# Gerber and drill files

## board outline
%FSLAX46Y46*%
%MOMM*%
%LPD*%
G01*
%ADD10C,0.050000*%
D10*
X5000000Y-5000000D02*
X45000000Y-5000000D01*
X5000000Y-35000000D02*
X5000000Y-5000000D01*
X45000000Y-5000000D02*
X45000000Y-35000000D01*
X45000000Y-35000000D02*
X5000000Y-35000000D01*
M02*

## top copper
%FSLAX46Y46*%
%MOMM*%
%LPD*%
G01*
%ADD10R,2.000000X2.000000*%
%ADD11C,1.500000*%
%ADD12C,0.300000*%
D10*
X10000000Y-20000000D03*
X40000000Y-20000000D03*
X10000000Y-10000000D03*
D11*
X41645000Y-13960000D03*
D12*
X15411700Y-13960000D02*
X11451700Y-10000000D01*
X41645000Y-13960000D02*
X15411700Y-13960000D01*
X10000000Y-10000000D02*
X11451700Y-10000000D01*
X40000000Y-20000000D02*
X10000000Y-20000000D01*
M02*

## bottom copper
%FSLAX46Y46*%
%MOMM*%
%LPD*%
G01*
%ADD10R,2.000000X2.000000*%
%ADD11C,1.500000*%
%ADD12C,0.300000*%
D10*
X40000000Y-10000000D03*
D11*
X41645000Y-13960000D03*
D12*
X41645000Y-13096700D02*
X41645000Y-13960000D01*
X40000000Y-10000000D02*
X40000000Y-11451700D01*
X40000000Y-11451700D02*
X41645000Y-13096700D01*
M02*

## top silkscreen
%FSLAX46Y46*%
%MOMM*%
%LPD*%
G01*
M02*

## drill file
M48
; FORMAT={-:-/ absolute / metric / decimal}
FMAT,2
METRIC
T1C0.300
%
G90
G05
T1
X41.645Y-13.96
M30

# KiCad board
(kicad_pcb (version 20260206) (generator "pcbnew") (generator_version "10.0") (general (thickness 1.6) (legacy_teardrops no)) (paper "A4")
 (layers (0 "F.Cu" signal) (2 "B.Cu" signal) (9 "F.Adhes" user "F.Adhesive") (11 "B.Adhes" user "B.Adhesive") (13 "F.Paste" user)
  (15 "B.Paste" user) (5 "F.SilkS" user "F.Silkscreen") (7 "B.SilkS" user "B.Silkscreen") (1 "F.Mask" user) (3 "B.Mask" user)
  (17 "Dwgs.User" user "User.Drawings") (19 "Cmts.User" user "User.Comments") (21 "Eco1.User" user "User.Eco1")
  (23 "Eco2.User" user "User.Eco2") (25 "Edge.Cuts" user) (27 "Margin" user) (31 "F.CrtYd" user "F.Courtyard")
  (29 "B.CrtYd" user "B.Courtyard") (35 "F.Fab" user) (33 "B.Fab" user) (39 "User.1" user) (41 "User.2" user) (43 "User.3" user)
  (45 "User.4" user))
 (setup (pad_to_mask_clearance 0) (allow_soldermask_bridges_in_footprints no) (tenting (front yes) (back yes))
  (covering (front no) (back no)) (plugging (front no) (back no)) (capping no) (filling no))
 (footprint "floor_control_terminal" (layer "F.Cu") (at 10 20)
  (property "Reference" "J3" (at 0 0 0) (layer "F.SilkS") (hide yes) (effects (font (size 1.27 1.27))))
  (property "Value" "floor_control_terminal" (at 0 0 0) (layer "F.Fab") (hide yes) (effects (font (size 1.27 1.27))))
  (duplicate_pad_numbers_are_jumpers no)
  (pad "1" smd rect (at 0 0) (size 2 2) (layers "F.Cu" "F.Mask" "F.Paste") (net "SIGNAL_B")))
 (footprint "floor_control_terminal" (layer "F.Cu") (at 40 20)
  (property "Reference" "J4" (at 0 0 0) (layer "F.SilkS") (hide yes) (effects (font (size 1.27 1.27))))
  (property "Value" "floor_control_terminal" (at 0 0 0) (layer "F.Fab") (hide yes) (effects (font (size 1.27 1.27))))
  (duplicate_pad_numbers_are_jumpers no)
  (pad "1" smd rect (at 0 0) (size 2 2) (layers "F.Cu" "F.Mask" "F.Paste") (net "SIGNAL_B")))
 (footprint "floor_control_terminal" (layer "F.Cu") (at 10 10)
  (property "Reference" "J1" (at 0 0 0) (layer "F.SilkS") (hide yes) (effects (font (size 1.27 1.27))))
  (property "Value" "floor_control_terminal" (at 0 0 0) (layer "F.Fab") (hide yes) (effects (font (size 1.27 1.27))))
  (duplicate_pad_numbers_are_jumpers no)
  (pad "1" smd rect (at 0 0) (size 2 2) (layers "F.Cu" "F.Mask" "F.Paste") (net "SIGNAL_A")))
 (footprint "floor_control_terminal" (layer "B.Cu") (at 40 10)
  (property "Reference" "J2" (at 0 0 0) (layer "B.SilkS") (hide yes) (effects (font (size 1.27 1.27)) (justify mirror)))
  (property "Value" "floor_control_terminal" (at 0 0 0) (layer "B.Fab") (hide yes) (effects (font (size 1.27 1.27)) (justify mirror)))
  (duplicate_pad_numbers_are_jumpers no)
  (pad "1" smd rect (at 0 0) (size 2 2) (layers "B.Cu" "B.Mask" "B.Paste") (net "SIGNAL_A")))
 (gr_line (start 5 5) (end 45 5) (stroke (width 0.05) (type default)) (layer "Edge.Cuts"))
 (gr_line (start 5 35) (end 5 5) (stroke (width 0.05) (type default)) (layer "Edge.Cuts"))
 (gr_line (start 45 5) (end 45 35) (stroke (width 0.05) (type default)) (layer "Edge.Cuts"))
 (gr_line (start 45 35) (end 5 35) (stroke (width 0.05) (type default)) (layer "Edge.Cuts"))
 (segment (start 15.4117 13.96) (end 11.4517 10) (width 0.3) (layer "F.Cu") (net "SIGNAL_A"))
 (segment (start 41.645 13.96) (end 15.4117 13.96) (width 0.3) (layer "F.Cu") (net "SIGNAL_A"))
 (segment (start 10 10) (end 11.4517 10) (width 0.3) (layer "F.Cu") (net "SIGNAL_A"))
 (via (at 41.645 13.96) (size 1.5) (drill 0.3) (layers "F.Cu" "B.Cu") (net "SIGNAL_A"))
 (segment (start 41.645 13.0967) (end 41.645 13.96) (width 0.3) (layer "B.Cu") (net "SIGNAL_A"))
 (segment (start 40 10) (end 40 11.4517) (width 0.3) (layer "B.Cu") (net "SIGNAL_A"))
 (segment (start 40 11.4517) (end 41.645 13.0967) (width 0.3) (layer "B.Cu") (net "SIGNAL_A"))
 (segment (start 40 20) (end 10 20) (width 0.3) (layer "F.Cu") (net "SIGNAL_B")))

